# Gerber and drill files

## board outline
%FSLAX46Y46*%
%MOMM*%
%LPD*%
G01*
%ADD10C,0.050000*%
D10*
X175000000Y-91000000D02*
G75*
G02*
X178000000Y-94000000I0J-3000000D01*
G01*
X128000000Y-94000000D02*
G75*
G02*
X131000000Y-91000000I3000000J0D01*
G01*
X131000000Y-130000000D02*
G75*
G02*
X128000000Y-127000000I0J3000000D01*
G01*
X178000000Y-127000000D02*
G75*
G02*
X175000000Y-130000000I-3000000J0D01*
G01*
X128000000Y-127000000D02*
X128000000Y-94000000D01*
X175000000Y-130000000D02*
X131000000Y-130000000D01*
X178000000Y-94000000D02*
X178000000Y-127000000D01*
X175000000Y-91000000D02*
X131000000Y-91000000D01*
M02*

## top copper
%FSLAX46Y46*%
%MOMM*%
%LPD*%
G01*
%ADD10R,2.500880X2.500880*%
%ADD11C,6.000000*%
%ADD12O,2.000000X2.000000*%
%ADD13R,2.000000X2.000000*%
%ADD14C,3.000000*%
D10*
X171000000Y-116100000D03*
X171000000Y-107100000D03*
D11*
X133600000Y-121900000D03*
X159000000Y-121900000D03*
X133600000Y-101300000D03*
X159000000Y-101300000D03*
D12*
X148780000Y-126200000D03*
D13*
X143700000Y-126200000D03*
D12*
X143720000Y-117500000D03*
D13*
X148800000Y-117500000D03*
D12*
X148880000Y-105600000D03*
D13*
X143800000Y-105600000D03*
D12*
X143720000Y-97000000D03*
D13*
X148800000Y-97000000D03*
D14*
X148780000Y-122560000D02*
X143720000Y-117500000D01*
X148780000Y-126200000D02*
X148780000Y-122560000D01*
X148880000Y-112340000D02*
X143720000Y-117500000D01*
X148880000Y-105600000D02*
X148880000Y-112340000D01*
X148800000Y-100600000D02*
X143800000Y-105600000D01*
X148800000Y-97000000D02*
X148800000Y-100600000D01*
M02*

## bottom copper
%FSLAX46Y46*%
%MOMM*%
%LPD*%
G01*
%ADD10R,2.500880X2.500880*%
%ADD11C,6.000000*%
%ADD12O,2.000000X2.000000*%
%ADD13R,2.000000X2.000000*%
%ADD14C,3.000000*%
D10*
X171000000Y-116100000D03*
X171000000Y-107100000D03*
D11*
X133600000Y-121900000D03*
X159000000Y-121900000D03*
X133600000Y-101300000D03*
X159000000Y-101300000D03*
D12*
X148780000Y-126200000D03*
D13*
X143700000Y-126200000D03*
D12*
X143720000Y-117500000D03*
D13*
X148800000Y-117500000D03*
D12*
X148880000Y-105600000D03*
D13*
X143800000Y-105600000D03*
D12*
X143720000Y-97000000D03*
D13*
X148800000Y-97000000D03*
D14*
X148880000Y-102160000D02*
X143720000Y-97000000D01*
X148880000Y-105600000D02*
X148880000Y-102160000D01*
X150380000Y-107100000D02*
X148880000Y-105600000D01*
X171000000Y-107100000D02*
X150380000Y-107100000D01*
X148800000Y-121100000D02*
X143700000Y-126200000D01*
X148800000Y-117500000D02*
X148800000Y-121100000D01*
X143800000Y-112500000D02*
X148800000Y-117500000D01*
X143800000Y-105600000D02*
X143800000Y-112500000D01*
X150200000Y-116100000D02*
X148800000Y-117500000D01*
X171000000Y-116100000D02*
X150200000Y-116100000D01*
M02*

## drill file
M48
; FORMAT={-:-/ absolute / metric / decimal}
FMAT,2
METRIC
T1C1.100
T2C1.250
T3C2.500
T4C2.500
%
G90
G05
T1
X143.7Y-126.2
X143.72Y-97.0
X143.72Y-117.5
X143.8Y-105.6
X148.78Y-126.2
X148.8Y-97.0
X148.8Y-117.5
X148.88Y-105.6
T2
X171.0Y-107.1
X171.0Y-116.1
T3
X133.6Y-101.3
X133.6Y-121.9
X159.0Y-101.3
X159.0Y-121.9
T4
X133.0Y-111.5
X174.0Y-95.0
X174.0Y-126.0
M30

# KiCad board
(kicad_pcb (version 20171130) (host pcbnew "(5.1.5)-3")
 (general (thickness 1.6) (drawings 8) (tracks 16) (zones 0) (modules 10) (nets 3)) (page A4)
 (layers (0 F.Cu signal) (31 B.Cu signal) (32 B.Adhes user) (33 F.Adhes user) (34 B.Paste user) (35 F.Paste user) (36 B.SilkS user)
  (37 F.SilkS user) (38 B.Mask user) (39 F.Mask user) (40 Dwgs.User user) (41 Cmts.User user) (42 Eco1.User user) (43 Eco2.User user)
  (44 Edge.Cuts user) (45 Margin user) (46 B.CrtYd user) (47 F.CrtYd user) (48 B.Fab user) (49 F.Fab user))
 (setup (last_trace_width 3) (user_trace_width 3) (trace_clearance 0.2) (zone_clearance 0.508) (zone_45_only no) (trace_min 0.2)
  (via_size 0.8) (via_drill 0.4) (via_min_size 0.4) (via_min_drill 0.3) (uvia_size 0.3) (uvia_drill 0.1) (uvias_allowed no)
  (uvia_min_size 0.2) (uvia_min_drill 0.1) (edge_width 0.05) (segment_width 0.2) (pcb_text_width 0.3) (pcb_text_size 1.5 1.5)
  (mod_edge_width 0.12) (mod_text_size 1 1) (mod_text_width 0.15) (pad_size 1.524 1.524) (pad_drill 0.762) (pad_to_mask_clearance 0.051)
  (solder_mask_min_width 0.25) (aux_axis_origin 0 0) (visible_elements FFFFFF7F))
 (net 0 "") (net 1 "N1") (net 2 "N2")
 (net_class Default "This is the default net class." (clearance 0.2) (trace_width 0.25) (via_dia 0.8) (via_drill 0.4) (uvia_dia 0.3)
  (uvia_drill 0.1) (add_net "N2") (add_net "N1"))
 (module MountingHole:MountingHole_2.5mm (layer F.Cu) (at 133 111.5)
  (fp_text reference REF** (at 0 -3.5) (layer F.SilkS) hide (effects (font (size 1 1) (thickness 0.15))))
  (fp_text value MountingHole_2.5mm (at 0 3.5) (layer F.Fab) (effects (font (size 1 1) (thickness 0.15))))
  (pad 1 np_thru_hole circle (at 0 0) (size 2.5 2.5) (drill 2.5) (layers *.Cu *.Mask)))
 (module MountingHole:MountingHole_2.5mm (layer F.Cu) (at 174 126)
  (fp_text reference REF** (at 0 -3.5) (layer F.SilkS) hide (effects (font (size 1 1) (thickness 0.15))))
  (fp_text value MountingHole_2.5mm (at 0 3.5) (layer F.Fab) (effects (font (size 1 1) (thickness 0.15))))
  (pad 1 np_thru_hole circle (at 0 0) (size 2.5 2.5) (drill 2.5) (layers *.Cu *.Mask)))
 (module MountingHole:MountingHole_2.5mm (layer F.Cu) (at 174 95)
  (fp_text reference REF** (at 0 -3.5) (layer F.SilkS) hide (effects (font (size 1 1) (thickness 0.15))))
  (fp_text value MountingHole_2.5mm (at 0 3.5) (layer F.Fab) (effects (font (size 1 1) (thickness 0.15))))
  (pad 1 np_thru_hole circle (at 0 0) (size 2.5 2.5) (drill 2.5) (layers *.Cu *.Mask)))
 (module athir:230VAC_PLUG (layer F.Cu) (at 171 111.6 270)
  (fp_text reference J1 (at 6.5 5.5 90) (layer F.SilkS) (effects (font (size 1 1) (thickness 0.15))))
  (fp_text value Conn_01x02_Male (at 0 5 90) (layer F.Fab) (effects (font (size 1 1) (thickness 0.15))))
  (pad 2 thru_hole rect (at 4.5 0 270) (size 2.50088 2.50088) (drill 1.25) (layers *.Cu *.Mask) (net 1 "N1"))
  (pad 1 thru_hole rect (at -4.5 0 270) (size 2.50088 2.50088) (drill 1.25) (layers *.Cu *.Mask) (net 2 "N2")))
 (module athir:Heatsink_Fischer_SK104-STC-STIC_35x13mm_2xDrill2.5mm (layer F.Cu) (at 146.3 121.9)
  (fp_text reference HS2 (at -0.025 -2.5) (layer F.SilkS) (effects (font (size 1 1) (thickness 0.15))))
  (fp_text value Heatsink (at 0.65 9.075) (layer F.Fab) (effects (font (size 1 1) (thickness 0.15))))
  (pad 1 thru_hole circle (at -12.7 0 180) (size 6 6) (drill 2.5) (layers *.Cu *.Mask))
  (pad 1 thru_hole circle (at 12.7 0) (size 6 6) (drill 2.5) (layers *.Cu *.Mask)))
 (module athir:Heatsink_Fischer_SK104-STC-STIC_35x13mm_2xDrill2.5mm (layer F.Cu) (at 146.3 101.3)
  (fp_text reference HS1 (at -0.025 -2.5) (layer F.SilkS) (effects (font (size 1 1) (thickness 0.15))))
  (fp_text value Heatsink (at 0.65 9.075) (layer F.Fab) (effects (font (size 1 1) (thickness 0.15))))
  (pad 1 thru_hole circle (at -12.7 0 180) (size 6 6) (drill 2.5) (layers *.Cu *.Mask))
  (pad 1 thru_hole circle (at 12.7 0) (size 6 6) (drill 2.5) (layers *.Cu *.Mask)))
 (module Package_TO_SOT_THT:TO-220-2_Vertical (layer F.Cu) (at 143.7 126.2)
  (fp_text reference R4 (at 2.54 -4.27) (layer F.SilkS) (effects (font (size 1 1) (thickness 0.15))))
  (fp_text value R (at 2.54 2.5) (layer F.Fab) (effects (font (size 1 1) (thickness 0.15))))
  (pad 2 thru_hole oval (at 5.08 0) (size 2 2) (drill 1.1) (layers *.Cu *.Mask) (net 2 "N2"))
  (pad 1 thru_hole rect (at 0 0) (size 2 2) (drill 1.1) (layers *.Cu *.Mask) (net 1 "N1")))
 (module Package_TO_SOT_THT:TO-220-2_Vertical (layer F.Cu) (at 148.8 117.5 180)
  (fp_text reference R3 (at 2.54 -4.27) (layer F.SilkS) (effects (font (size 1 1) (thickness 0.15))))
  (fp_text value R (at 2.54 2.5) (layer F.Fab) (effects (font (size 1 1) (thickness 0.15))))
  (pad 2 thru_hole oval (at 5.08 0 180) (size 2 2) (drill 1.1) (layers *.Cu *.Mask) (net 2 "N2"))
  (pad 1 thru_hole rect (at 0 0 180) (size 2 2) (drill 1.1) (layers *.Cu *.Mask) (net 1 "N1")))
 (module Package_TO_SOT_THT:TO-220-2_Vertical (layer F.Cu) (at 143.8 105.6)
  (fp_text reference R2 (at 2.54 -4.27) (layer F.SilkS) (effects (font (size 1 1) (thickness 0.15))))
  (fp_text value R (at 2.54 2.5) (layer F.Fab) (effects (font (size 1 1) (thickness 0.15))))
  (pad 2 thru_hole oval (at 5.08 0) (size 2 2) (drill 1.1) (layers *.Cu *.Mask) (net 2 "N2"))
  (pad 1 thru_hole rect (at 0 0) (size 2 2) (drill 1.1) (layers *.Cu *.Mask) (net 1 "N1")))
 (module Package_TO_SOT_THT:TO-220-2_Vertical (layer F.Cu) (at 148.8 97 180)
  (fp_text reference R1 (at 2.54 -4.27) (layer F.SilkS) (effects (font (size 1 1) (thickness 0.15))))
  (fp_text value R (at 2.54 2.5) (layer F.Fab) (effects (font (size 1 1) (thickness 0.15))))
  (pad 2 thru_hole oval (at 5.08 0 180) (size 2 2) (drill 1.1) (layers *.Cu *.Mask) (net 2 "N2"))
  (pad 1 thru_hole rect (at 0 0 180) (size 2 2) (drill 1.1) (layers *.Cu *.Mask) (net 1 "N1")))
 (gr_arc (start 175 94) (end 178 94) (angle -90) (layer Edge.Cuts) (width 0.05))
 (gr_arc (start 131 94) (end 131 91) (angle -90) (layer Edge.Cuts) (width 0.05))
 (gr_arc (start 131 127) (end 128 127) (angle -90) (layer Edge.Cuts) (width 0.05))
 (gr_arc (start 175 127) (end 175 130) (angle -90) (layer Edge.Cuts) (width 0.05))
 (gr_line (start 128 127) (end 128 94) (layer Edge.Cuts) (width 0.05))
 (gr_line (start 175 130) (end 131 130) (layer Edge.Cuts) (width 0.05))
 (gr_line (start 178 94) (end 178 127) (layer Edge.Cuts) (width 0.05))
 (gr_line (start 175 91) (end 131 91) (layer Edge.Cuts) (width 0.05))
 (segment (start 148.78 122.56) (end 143.72 117.5) (width 3) (layer F.Cu) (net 2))
 (segment (start 148.78 126.2) (end 148.78 122.56) (width 3) (layer F.Cu) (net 2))
 (segment (start 148.88 102.16) (end 143.72 97) (width 3) (layer B.Cu) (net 2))
 (segment (start 148.88 105.6) (end 148.88 102.16) (width 3) (layer B.Cu) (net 2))
 (segment (start 148.88 112.34) (end 143.72 117.5) (width 3) (layer F.Cu) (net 2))
 (segment (start 148.88 105.6) (end 148.88 112.34) (width 3) (layer F.Cu) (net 2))
 (segment (start 150.38 107.1) (end 148.88 105.6) (width 3) (layer B.Cu) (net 2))
 (segment (start 171 107.1) (end 150.38 107.1) (width 3) (layer B.Cu) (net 2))
 (segment (start 148.8 121.1) (end 143.7 126.2) (width 3) (layer B.Cu) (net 1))
 (segment (start 148.8 117.5) (end 148.8 121.1) (width 3) (layer B.Cu) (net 1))
 (segment (start 148.8 100.6) (end 143.8 105.6) (width 3) (layer F.Cu) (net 1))
 (segment (start 148.8 97) (end 148.8 100.6) (width 3) (layer F.Cu) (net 1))
 (segment (start 143.8 112.5) (end 148.8 117.5) (width 3) (layer B.Cu) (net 1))
 (segment (start 143.8 105.6) (end 143.8 112.5) (width 3) (layer B.Cu) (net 1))
 (segment (start 150.2 116.1) (end 148.8 117.5) (width 3) (layer B.Cu) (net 1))
 (segment (start 171 116.1) (end 150.2 116.1) (width 3) (layer B.Cu) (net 1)))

